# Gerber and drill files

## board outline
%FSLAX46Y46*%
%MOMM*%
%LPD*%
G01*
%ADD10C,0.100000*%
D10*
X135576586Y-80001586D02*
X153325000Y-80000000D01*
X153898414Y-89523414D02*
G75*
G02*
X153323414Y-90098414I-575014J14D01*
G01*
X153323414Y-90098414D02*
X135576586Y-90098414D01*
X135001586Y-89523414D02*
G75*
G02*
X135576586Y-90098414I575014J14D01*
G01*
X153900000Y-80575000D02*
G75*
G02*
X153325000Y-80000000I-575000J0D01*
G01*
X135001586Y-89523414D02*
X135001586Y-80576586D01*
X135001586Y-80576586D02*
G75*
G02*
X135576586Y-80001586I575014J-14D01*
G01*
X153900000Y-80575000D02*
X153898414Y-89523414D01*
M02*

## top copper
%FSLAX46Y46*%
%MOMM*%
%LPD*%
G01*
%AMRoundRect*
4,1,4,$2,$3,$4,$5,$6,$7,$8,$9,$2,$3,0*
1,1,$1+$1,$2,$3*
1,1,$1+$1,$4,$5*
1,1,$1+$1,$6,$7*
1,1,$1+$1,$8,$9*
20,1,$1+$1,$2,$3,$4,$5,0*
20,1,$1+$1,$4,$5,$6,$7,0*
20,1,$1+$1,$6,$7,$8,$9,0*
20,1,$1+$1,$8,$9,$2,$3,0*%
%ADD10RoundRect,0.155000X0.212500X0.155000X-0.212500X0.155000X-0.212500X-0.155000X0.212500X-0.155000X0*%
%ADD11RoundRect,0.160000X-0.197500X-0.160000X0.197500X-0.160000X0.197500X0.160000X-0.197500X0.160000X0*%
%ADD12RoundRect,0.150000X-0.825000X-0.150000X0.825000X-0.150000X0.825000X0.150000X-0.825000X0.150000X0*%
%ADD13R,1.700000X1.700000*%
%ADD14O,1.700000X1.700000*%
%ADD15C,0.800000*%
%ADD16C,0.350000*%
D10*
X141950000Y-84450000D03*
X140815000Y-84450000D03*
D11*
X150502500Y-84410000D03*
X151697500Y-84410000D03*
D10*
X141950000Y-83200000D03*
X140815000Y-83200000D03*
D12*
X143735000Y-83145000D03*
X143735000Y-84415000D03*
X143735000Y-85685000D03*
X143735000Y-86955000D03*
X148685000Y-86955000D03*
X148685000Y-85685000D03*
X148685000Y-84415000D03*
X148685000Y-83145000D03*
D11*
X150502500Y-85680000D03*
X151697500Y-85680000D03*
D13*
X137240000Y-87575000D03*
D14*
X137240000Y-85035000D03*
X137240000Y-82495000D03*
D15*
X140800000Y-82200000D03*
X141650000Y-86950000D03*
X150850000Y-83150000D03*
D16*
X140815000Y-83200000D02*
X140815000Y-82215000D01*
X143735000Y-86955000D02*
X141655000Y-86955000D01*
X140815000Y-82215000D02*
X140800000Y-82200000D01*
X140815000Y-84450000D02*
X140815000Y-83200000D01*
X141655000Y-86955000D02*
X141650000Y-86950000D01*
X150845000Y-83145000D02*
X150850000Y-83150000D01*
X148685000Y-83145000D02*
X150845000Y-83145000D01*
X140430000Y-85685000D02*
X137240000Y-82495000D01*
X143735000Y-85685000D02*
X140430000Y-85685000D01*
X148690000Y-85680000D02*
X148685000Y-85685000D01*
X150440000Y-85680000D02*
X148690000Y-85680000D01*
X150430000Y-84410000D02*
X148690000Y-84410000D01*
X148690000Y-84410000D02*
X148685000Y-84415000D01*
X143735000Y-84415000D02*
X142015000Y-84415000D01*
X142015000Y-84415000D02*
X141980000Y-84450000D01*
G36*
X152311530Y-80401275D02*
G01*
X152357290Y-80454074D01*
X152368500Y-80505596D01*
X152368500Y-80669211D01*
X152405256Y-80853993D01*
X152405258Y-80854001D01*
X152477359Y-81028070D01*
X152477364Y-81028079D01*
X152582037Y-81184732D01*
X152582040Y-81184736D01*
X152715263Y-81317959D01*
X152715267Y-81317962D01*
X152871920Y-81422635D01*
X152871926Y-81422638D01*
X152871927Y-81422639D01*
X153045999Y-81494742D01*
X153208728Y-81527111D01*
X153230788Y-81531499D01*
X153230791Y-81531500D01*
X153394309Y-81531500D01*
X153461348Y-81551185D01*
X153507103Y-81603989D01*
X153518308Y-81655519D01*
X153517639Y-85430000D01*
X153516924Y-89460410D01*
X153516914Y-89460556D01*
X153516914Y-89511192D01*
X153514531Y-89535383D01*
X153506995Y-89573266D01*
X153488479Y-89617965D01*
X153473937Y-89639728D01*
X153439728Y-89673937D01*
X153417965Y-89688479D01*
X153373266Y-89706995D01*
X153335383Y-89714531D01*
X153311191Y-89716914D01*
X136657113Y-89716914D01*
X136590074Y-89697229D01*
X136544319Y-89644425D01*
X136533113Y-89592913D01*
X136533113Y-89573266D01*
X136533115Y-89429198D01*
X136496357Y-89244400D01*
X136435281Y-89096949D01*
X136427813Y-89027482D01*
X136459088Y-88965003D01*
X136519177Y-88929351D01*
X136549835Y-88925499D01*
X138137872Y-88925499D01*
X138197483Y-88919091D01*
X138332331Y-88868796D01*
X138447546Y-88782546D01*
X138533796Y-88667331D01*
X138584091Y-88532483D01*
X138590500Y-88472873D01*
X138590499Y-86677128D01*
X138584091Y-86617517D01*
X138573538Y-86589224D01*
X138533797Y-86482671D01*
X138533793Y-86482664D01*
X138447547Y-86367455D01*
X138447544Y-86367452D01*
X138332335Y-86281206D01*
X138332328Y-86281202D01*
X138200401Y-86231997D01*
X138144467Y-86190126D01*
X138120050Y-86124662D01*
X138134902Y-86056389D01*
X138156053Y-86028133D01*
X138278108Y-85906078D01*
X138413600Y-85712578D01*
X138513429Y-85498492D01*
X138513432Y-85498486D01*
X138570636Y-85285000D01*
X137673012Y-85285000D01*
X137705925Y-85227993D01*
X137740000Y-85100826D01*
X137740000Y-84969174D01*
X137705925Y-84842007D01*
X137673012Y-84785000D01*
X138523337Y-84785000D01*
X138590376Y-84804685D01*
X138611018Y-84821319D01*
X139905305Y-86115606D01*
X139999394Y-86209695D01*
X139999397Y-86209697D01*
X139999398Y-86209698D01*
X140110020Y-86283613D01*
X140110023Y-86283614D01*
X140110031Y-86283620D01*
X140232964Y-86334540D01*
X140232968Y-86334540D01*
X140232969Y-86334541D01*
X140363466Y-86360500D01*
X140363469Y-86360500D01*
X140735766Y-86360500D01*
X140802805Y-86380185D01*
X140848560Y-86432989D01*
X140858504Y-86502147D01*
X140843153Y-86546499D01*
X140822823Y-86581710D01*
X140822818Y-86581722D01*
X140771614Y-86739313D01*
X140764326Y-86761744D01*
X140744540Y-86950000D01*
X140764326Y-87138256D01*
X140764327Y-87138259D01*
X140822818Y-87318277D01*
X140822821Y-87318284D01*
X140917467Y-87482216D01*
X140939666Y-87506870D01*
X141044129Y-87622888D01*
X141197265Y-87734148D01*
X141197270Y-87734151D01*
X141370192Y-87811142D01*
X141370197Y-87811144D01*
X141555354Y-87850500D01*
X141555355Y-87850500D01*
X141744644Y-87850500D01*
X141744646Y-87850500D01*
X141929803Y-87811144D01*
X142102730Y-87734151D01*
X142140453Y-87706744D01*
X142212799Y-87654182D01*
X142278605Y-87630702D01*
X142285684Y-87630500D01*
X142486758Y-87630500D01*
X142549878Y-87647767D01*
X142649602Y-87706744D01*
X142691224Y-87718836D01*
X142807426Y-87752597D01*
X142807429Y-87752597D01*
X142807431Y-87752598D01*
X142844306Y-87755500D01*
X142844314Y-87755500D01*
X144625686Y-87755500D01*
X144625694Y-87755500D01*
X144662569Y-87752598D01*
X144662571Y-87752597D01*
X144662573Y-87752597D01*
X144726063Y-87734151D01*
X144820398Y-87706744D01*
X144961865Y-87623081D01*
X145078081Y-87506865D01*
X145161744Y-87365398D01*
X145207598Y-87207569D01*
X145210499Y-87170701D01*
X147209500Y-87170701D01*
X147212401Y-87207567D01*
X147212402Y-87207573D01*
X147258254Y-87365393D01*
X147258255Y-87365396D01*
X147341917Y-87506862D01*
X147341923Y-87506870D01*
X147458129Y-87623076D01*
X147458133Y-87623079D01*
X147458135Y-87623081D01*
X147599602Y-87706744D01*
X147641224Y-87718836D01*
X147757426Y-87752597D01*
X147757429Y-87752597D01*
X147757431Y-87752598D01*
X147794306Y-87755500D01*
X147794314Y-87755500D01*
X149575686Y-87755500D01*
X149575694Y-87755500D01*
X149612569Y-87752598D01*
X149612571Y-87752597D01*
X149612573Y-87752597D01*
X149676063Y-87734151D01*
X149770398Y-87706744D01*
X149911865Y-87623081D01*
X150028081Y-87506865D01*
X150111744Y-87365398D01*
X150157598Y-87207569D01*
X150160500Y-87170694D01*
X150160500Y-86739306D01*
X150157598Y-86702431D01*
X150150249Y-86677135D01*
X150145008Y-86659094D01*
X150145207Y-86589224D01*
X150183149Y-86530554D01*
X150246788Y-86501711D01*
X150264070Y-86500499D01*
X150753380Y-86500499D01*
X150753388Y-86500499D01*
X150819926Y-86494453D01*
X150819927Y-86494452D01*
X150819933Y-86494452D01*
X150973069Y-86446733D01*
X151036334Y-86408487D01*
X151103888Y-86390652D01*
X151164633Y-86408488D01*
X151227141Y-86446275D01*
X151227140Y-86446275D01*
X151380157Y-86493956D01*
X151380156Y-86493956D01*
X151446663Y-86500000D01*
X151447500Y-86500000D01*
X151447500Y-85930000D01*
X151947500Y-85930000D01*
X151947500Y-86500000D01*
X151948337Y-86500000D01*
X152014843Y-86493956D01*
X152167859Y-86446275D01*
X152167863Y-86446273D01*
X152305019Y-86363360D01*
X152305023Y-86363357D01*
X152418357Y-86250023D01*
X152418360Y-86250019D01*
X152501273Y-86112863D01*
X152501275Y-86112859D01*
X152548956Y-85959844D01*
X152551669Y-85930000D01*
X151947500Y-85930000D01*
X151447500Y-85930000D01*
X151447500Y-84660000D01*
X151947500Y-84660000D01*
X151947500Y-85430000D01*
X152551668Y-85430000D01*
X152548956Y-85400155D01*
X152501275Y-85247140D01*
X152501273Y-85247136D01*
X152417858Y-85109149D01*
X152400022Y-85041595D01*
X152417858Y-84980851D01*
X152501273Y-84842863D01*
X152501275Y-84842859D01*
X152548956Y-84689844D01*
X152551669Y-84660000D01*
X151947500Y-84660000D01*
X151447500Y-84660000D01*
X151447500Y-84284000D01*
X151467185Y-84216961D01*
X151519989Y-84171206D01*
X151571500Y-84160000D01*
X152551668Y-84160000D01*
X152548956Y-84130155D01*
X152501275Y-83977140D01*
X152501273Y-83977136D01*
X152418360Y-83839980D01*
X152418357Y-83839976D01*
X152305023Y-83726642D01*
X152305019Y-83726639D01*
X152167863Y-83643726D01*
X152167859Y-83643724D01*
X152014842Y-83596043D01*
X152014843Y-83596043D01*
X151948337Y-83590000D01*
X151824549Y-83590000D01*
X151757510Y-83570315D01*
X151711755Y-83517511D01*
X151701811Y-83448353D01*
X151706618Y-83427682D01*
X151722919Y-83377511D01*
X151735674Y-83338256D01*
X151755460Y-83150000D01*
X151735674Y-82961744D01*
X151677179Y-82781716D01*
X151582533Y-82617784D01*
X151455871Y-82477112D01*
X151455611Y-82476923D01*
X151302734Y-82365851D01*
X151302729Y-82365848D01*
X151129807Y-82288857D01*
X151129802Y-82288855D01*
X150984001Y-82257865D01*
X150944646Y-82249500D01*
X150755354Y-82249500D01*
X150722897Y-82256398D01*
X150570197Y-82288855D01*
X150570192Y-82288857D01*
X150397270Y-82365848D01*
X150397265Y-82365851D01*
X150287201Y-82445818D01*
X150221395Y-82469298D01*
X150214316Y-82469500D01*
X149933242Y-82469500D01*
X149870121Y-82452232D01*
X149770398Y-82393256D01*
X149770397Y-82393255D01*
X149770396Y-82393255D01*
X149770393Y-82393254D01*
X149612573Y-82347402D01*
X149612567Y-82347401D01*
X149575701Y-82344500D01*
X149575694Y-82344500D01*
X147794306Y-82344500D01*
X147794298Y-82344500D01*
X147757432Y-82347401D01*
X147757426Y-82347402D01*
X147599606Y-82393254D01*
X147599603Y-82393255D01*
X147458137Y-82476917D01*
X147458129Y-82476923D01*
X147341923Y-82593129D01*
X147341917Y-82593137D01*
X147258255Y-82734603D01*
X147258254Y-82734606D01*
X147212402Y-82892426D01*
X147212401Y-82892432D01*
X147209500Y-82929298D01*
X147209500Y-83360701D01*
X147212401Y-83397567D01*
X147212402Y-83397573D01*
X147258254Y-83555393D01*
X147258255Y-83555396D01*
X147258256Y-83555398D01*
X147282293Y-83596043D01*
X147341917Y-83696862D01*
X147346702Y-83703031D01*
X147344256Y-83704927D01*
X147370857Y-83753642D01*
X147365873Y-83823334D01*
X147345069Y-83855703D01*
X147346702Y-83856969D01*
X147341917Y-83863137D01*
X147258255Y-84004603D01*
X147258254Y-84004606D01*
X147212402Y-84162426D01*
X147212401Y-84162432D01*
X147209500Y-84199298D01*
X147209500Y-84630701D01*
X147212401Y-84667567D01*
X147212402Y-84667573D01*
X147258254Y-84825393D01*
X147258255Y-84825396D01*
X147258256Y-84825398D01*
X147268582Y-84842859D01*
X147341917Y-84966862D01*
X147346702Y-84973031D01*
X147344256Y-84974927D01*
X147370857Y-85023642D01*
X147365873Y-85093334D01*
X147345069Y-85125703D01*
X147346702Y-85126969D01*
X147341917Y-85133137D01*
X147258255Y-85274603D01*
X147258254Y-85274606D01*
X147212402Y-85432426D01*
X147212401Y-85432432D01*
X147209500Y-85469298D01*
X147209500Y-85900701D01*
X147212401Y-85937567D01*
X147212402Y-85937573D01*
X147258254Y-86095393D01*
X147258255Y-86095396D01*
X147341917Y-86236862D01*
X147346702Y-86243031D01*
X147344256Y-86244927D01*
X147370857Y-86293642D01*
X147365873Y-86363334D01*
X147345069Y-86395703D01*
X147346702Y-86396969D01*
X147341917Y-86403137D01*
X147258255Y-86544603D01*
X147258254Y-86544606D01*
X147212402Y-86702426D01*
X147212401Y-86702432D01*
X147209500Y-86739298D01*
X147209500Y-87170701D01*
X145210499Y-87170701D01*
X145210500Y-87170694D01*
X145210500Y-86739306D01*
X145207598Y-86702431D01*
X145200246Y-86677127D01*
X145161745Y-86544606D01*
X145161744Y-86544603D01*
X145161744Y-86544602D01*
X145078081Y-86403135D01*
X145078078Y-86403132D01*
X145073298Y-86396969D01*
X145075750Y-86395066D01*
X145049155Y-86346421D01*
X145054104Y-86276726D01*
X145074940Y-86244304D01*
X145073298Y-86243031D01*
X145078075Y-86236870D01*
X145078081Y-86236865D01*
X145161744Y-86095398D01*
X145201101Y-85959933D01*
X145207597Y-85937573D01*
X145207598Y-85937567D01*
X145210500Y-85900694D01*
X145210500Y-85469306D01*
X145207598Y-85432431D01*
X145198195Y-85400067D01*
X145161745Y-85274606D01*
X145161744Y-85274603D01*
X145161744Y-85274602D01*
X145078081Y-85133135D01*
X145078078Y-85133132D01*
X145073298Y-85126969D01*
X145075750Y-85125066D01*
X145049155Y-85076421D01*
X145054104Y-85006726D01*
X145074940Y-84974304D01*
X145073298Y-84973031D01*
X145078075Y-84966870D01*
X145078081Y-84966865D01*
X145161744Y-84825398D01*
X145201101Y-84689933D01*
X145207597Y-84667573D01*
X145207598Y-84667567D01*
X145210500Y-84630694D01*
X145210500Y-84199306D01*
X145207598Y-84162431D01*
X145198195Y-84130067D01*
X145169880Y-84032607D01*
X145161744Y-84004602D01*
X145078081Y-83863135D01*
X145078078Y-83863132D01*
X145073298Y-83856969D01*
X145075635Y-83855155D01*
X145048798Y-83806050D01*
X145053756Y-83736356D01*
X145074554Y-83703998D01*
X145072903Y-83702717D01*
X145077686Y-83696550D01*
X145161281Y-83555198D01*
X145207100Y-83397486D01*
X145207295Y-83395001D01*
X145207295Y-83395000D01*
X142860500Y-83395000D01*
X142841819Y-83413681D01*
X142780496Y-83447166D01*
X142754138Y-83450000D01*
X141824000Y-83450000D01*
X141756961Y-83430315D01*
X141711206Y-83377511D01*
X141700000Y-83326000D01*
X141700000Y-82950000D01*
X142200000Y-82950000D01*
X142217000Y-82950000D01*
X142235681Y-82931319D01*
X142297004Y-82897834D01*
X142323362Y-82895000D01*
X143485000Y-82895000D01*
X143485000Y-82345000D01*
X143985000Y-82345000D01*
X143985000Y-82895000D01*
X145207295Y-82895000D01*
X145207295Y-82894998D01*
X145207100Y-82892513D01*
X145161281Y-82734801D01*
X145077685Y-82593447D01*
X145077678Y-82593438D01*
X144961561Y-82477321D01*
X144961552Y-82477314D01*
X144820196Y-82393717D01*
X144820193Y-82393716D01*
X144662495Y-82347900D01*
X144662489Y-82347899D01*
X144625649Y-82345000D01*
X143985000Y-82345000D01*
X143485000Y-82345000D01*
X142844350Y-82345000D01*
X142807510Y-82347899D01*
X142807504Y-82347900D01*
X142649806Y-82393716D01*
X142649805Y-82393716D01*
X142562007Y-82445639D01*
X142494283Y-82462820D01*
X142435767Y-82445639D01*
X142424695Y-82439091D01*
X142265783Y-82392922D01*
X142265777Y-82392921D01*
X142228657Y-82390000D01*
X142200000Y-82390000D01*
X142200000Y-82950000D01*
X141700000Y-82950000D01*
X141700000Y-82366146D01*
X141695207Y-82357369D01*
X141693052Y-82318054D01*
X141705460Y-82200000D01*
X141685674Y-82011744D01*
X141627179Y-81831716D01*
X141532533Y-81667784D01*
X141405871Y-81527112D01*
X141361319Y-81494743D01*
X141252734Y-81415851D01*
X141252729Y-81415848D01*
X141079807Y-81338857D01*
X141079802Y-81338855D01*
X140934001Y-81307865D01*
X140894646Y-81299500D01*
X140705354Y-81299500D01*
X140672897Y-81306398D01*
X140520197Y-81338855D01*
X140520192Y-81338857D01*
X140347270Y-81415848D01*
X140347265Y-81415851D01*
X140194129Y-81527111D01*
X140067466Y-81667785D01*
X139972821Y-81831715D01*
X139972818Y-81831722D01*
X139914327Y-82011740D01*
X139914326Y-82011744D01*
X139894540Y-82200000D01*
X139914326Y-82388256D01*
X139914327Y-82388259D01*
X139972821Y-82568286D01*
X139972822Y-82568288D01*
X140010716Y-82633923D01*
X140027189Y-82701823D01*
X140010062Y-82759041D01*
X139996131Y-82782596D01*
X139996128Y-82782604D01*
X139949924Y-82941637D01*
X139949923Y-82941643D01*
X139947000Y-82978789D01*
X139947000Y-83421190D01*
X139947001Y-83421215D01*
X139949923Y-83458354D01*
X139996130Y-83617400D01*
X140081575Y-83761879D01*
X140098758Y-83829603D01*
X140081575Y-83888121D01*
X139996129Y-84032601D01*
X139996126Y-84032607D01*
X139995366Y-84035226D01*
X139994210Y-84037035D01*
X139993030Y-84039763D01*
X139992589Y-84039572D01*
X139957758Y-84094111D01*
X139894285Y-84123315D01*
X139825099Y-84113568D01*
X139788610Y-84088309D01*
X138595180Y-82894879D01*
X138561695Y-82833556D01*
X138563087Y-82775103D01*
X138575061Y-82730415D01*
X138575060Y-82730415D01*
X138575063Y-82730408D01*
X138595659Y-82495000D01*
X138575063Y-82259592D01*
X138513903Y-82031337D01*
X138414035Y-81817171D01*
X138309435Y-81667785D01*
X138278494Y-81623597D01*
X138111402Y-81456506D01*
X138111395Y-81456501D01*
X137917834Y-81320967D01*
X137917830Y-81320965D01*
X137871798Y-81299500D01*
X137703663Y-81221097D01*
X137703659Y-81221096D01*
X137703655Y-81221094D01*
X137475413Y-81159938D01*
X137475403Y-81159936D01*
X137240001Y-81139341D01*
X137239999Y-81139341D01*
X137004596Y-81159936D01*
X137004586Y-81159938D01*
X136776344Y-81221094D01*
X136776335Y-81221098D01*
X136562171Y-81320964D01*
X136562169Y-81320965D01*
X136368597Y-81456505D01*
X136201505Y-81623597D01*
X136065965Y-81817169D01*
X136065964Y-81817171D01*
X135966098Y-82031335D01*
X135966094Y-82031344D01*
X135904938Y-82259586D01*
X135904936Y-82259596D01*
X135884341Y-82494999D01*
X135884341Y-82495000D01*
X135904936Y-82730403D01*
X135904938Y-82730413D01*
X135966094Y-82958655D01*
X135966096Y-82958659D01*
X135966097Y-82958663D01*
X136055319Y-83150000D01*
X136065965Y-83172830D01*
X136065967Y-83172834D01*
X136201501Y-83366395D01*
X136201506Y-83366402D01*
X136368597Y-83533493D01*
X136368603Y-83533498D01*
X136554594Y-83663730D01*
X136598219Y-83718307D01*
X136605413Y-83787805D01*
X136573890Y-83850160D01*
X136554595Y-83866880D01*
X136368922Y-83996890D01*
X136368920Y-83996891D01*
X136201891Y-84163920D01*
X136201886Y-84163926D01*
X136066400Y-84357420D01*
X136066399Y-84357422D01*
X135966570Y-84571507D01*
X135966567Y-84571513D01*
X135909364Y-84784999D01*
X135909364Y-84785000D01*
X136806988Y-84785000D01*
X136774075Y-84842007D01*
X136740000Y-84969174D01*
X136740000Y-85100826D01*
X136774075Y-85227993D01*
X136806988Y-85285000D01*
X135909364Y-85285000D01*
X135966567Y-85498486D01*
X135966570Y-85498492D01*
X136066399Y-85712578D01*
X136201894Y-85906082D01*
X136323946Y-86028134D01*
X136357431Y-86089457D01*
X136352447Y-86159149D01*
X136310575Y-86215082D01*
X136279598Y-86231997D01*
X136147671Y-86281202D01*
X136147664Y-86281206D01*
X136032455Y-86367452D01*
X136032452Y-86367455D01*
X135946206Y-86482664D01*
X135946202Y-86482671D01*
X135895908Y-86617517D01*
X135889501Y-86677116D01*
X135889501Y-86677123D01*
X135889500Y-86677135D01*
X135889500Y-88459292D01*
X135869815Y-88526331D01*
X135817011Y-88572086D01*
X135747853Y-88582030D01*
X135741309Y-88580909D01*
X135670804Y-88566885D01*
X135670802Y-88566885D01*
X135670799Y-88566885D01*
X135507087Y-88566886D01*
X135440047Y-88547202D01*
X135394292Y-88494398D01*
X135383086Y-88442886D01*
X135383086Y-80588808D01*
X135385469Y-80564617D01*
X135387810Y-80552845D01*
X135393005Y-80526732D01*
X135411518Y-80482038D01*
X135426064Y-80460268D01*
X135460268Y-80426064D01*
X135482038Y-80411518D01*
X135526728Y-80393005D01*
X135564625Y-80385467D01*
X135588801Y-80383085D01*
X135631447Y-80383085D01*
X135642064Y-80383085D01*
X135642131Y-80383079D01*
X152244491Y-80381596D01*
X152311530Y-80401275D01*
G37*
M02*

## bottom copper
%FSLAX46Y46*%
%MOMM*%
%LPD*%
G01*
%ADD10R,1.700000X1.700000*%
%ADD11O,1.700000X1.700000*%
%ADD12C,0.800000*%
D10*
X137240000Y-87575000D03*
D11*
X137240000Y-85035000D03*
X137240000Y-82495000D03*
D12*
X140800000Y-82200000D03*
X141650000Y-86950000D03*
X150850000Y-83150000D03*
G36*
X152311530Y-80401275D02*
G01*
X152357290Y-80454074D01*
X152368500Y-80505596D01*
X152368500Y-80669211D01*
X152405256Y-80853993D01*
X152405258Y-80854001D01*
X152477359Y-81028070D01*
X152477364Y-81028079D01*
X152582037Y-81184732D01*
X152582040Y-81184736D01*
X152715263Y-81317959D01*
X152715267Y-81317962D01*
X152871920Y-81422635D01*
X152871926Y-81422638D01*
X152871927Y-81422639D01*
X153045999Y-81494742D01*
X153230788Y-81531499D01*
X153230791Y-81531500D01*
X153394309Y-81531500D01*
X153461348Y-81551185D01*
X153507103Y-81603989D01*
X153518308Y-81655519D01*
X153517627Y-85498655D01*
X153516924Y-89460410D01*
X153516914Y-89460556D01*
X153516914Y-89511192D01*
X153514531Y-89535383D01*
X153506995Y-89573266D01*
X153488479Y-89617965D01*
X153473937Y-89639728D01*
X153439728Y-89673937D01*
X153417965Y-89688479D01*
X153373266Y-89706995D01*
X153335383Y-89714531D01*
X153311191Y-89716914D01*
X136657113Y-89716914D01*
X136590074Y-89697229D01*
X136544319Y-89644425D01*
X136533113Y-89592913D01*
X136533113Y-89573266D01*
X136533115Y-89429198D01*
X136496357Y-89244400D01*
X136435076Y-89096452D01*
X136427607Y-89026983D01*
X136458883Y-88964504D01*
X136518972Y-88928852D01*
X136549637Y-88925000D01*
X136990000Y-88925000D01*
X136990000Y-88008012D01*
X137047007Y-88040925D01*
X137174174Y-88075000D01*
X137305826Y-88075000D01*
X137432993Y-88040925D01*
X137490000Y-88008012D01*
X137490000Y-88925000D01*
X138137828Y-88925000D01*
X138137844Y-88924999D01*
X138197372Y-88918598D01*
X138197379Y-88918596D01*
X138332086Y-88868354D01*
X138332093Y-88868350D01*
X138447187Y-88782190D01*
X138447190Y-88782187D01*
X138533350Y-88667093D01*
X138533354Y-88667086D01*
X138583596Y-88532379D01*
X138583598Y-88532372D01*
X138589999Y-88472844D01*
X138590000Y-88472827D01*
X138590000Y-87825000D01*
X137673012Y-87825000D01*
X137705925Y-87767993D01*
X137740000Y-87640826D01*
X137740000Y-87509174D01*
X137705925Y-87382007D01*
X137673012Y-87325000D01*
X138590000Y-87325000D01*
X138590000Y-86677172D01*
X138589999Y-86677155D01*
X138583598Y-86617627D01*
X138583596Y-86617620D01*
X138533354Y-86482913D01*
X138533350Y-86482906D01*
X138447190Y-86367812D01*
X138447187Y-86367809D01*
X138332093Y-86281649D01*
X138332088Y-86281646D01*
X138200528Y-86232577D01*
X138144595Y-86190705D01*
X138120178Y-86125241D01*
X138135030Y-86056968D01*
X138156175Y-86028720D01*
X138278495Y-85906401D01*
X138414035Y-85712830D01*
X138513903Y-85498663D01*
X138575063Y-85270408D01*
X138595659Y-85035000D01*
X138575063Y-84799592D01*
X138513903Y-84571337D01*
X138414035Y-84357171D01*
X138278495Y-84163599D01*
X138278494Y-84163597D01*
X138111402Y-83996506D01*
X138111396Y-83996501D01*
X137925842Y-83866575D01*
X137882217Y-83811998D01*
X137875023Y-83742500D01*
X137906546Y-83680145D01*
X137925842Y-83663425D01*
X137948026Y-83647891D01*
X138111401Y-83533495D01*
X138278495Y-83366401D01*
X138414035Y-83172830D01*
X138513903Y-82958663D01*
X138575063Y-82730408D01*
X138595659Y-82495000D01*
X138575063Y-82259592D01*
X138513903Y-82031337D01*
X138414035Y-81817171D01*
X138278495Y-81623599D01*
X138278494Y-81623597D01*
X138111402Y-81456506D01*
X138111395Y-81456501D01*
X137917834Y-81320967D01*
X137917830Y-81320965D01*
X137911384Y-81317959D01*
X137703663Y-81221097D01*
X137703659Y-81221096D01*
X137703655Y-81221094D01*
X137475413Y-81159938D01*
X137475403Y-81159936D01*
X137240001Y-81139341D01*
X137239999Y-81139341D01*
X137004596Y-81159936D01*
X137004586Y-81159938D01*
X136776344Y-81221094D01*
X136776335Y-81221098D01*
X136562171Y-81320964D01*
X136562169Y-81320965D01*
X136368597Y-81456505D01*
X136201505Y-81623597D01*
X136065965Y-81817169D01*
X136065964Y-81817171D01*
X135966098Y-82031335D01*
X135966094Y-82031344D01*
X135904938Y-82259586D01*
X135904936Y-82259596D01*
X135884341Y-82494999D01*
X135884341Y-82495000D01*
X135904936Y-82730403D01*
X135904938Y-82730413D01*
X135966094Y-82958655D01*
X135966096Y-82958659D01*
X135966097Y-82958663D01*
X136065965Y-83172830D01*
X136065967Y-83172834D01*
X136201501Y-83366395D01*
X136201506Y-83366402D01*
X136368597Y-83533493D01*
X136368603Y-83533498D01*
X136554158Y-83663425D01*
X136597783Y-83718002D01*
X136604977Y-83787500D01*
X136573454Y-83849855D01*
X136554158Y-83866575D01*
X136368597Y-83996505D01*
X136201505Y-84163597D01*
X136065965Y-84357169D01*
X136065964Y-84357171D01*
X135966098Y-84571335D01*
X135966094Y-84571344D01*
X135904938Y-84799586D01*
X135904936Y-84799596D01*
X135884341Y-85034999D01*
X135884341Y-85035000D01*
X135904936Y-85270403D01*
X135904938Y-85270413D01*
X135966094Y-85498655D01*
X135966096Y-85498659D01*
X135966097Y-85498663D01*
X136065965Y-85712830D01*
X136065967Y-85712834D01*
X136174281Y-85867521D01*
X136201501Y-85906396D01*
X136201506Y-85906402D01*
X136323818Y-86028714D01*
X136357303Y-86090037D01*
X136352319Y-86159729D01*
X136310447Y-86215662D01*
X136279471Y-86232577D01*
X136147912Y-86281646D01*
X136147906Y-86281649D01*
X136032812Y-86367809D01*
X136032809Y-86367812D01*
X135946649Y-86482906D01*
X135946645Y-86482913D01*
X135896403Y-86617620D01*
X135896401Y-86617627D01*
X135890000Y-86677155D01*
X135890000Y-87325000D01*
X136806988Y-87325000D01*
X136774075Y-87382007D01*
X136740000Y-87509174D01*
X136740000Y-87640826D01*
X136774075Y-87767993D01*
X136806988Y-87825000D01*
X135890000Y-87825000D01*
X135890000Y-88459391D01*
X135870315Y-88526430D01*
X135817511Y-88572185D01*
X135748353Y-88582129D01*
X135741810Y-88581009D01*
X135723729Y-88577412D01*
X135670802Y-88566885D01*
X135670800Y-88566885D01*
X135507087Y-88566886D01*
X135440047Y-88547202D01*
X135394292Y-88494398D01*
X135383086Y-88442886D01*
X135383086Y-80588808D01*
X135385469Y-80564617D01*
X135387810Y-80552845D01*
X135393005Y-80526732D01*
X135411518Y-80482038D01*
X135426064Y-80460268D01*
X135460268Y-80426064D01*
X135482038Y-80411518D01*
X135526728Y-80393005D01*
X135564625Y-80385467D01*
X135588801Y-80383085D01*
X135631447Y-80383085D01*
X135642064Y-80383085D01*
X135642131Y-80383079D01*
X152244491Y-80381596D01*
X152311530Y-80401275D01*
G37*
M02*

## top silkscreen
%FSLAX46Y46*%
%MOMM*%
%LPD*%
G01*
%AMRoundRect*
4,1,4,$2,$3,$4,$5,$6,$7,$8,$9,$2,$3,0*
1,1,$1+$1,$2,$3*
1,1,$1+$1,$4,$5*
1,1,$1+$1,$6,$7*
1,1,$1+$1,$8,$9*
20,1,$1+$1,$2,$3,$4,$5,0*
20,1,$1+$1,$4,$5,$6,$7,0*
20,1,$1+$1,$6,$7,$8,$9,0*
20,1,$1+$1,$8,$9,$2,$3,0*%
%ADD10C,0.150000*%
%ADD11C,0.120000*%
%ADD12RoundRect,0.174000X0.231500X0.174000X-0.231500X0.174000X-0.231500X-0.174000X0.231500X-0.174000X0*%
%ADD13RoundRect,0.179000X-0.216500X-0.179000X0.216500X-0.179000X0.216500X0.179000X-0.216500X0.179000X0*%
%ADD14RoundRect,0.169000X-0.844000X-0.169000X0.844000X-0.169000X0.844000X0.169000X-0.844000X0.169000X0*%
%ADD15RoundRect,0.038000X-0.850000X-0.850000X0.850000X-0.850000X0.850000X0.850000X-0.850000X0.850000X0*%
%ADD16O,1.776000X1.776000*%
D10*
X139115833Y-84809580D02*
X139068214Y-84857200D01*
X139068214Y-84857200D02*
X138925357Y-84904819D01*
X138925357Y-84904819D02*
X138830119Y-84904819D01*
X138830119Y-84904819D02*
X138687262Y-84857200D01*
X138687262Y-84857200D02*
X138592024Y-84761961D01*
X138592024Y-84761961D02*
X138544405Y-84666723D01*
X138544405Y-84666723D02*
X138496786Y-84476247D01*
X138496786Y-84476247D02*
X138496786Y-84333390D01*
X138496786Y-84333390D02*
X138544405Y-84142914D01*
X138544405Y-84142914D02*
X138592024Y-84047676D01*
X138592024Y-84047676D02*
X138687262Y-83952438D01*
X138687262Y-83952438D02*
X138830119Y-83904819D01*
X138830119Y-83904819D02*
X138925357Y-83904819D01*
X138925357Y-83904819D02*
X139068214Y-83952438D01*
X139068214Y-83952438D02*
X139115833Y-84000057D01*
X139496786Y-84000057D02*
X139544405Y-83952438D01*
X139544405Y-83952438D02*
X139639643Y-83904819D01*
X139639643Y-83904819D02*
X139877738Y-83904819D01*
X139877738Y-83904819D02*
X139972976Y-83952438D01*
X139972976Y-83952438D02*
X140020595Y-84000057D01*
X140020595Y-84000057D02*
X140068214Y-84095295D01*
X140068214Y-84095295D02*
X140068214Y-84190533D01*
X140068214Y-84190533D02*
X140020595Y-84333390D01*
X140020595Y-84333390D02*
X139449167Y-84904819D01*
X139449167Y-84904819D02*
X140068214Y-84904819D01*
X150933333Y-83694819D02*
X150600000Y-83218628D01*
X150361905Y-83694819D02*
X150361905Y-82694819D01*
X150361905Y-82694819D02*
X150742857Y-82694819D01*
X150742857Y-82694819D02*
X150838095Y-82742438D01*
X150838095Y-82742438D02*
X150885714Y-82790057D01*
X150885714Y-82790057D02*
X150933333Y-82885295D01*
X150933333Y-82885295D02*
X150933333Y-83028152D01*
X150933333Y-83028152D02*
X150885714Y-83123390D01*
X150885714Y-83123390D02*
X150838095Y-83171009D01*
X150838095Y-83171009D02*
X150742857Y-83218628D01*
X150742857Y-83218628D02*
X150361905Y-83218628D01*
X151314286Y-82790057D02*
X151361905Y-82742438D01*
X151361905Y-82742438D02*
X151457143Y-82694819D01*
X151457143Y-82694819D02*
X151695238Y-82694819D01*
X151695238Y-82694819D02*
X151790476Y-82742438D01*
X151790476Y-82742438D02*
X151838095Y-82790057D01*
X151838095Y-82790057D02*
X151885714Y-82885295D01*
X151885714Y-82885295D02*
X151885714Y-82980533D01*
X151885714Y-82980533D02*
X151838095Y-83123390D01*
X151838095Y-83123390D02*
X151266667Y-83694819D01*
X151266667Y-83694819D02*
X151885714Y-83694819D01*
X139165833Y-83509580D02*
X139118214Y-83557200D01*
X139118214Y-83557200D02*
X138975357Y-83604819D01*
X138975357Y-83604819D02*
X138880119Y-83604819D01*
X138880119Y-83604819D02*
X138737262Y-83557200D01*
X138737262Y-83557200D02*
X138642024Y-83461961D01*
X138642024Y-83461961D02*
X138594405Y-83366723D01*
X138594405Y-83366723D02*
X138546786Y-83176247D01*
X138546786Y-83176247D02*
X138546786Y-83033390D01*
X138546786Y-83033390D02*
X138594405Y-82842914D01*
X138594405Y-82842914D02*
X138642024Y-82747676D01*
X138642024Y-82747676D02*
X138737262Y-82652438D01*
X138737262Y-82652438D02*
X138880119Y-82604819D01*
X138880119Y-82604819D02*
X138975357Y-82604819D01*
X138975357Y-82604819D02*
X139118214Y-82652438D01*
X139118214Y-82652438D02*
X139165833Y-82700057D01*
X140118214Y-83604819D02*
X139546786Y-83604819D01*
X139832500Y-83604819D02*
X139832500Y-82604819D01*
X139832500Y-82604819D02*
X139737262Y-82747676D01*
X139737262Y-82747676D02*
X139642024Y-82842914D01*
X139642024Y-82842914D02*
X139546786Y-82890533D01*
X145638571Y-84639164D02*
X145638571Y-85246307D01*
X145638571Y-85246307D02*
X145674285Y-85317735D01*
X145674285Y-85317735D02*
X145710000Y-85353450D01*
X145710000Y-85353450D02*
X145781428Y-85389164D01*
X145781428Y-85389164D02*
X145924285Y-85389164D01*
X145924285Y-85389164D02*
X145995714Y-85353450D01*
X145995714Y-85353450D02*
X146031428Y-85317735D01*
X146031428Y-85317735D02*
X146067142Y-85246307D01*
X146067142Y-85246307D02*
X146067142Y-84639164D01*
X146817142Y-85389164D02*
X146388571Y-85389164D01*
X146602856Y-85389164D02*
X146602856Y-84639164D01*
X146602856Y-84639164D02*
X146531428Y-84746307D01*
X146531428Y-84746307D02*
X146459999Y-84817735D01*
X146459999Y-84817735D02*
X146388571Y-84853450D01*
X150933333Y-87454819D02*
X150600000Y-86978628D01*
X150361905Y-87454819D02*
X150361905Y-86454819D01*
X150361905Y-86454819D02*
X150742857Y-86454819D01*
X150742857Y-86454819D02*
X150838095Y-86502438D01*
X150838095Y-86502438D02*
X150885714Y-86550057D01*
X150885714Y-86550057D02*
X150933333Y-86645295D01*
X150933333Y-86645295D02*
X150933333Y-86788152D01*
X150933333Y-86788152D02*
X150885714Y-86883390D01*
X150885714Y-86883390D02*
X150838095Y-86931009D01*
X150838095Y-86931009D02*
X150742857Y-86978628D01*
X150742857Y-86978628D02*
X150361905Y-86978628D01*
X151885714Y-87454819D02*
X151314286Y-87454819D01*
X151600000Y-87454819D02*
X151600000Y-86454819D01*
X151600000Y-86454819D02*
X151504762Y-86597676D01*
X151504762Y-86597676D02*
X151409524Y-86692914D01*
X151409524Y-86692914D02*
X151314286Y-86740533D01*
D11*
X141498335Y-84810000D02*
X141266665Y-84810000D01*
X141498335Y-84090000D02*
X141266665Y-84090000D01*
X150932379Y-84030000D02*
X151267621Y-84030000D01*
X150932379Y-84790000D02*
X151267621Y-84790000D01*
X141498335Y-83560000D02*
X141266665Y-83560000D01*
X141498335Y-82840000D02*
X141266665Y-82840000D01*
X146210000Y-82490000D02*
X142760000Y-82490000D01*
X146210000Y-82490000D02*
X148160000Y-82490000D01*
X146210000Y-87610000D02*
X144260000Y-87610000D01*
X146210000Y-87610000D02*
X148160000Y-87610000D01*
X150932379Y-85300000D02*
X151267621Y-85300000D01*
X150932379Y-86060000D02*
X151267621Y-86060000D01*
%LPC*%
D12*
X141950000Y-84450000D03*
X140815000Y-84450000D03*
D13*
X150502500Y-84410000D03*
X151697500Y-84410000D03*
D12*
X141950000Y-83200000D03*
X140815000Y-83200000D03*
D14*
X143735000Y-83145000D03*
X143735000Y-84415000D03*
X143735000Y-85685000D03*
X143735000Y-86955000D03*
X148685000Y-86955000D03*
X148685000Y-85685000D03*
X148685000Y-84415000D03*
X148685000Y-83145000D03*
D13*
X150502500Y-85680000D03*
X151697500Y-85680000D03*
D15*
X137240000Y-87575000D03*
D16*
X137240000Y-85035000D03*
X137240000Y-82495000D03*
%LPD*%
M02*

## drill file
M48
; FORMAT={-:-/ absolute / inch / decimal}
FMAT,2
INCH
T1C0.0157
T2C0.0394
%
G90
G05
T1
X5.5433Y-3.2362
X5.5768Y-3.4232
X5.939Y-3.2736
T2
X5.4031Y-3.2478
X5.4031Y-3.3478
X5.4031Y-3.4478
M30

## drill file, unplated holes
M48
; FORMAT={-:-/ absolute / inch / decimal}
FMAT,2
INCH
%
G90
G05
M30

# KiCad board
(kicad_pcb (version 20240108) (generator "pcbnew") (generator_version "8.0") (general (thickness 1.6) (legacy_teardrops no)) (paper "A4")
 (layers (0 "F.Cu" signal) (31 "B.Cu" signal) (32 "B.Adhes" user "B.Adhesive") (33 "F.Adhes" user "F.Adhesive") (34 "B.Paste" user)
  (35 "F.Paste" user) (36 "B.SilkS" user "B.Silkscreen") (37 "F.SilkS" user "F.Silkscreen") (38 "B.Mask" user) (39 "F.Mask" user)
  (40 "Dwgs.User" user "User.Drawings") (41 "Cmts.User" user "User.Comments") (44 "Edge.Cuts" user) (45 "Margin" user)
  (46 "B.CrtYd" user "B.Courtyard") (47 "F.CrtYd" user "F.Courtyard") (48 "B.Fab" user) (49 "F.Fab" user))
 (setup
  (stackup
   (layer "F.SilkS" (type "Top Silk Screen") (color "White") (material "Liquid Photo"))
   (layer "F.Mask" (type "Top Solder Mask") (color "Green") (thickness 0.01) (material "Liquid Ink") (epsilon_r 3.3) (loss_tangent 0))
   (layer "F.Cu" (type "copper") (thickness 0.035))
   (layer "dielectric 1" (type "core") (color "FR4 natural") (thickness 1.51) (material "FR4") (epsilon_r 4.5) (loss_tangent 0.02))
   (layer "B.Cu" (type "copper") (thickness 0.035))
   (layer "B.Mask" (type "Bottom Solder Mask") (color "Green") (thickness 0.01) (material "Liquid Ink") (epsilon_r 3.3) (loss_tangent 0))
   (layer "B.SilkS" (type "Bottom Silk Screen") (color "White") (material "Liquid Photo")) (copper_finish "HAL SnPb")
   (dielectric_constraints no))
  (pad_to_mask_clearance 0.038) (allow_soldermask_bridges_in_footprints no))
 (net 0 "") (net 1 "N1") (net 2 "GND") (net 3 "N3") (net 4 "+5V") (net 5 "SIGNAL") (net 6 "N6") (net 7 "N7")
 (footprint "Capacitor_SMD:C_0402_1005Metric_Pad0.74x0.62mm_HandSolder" (layer "F.Cu") (at 141.3825 84.45 180)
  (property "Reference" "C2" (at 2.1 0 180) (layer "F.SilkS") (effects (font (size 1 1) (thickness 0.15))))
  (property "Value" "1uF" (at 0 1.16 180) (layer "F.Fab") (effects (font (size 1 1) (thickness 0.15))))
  (fp_line (start -0.115835 0.36) (end 0.115835 0.36) (stroke (width 0.12) (type solid)) (layer "F.SilkS"))
  (fp_line (start -0.115835 -0.36) (end 0.115835 -0.36) (stroke (width 0.12) (type solid)) (layer "F.SilkS"))
  (pad "1" smd roundrect (at -0.5675 0 180) (size 0.735 0.62) (layers "F.Cu" "F.Paste" "F.Mask") (roundrect_rratio 0.25) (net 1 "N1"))
  (pad "2" smd roundrect (at 0.5675 0 180) (size 0.735 0.62) (layers "F.Cu" "F.Paste" "F.Mask") (roundrect_rratio 0.25) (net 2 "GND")))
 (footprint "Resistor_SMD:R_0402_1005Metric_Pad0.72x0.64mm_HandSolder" (layer "F.Cu") (at 151.1 84.41)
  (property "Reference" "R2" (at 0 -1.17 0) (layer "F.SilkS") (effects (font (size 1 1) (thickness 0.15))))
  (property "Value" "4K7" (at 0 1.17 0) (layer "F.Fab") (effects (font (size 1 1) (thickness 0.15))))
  (fp_line (start -0.167621 -0.38) (end 0.167621 -0.38) (stroke (width 0.12) (type solid)) (layer "F.SilkS"))
  (fp_line (start -0.167621 0.38) (end 0.167621 0.38) (stroke (width 0.12) (type solid)) (layer "F.SilkS"))
  (pad "1" smd roundrect (at -0.5975 0) (size 0.715 0.64) (layers "F.Cu" "F.Paste" "F.Mask") (roundrect_rratio 0.25) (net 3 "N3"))
  (pad "2" smd roundrect (at 0.5975 0) (size 0.715 0.64) (layers "F.Cu" "F.Paste" "F.Mask") (roundrect_rratio 0.25) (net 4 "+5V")))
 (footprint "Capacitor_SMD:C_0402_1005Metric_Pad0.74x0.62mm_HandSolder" (layer "F.Cu") (at 141.3825 83.2 180)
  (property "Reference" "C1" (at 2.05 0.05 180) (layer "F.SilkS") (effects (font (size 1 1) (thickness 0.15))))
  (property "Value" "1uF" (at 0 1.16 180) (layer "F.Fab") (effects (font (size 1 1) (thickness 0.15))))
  (fp_line (start -0.115835 0.36) (end 0.115835 0.36) (stroke (width 0.12) (type solid)) (layer "F.SilkS"))
  (fp_line (start -0.115835 -0.36) (end 0.115835 -0.36) (stroke (width 0.12) (type solid)) (layer "F.SilkS"))
  (pad "1" smd roundrect (at -0.5675 0 180) (size 0.735 0.62) (layers "F.Cu" "F.Paste" "F.Mask") (roundrect_rratio 0.25) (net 4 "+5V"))
  (pad "2" smd roundrect (at 0.5675 0 180) (size 0.735 0.62) (layers "F.Cu" "F.Paste" "F.Mask") (roundrect_rratio 0.25) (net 2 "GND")))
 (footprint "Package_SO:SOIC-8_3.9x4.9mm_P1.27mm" (layer "F.Cu") (at 146.21 85.05)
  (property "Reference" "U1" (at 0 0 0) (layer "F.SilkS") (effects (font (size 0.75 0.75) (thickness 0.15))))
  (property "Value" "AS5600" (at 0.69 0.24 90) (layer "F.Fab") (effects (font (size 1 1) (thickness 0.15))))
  (fp_line (start 0 -2.56) (end -3.45 -2.56) (stroke (width 0.12) (type solid)) (layer "F.SilkS"))
  (fp_line (start 0 -2.56) (end 1.95 -2.56) (stroke (width 0.12) (type solid)) (layer "F.SilkS"))
  (fp_line (start 0 2.56) (end -1.95 2.56) (stroke (width 0.12) (type solid)) (layer "F.SilkS"))
  (fp_line (start 0 2.56) (end 1.95 2.56) (stroke (width 0.12) (type solid)) (layer "F.SilkS"))
  (pad "1" smd roundrect (at -2.475 -1.905) (size 1.95 0.6) (layers "F.Cu" "F.Paste" "F.Mask") (roundrect_rratio 0.25) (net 4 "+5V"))
  (pad "2" smd roundrect (at -2.475 -0.635) (size 1.95 0.6) (layers "F.Cu" "F.Paste" "F.Mask") (roundrect_rratio 0.25) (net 1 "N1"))
  (pad "3" smd roundrect (at -2.475 0.635) (size 1.95 0.6) (layers "F.Cu" "F.Paste" "F.Mask") (roundrect_rratio 0.25) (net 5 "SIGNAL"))
  (pad "4" smd roundrect (at -2.475 1.905) (size 1.95 0.6) (layers "F.Cu" "F.Paste" "F.Mask") (roundrect_rratio 0.25) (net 2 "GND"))
  (pad "5" smd roundrect (at 2.475 1.905) (size 1.95 0.6) (layers "F.Cu" "F.Paste" "F.Mask") (roundrect_rratio 0.25) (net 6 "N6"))
  (pad "6" smd roundrect (at 2.475 0.635) (size 1.95 0.6) (layers "F.Cu" "F.Paste" "F.Mask") (roundrect_rratio 0.25) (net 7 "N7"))
  (pad "7" smd roundrect (at 2.475 -0.635) (size 1.95 0.6) (layers "F.Cu" "F.Paste" "F.Mask") (roundrect_rratio 0.25) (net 3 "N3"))
  (pad "8" smd roundrect (at 2.475 -1.905) (size 1.95 0.6) (layers "F.Cu" "F.Paste" "F.Mask") (roundrect_rratio 0.25) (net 2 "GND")))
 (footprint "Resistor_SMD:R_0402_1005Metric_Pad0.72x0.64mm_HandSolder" (layer "F.Cu") (at 151.1 85.68)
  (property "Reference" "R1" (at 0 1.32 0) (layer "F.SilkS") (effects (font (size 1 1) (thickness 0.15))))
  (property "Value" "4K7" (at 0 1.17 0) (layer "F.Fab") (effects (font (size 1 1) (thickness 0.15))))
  (fp_line (start -0.167621 -0.38) (end 0.167621 -0.38) (stroke (width 0.12) (type solid)) (layer "F.SilkS"))
  (fp_line (start -0.167621 0.38) (end 0.167621 0.38) (stroke (width 0.12) (type solid)) (layer "F.SilkS"))
  (pad "1" smd roundrect (at -0.5975 0) (size 0.715 0.64) (layers "F.Cu" "F.Paste" "F.Mask") (roundrect_rratio 0.25) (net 7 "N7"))
  (pad "2" smd roundrect (at 0.5975 0) (size 0.715 0.64) (layers "F.Cu" "F.Paste" "F.Mask") (roundrect_rratio 0.25) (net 4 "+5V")))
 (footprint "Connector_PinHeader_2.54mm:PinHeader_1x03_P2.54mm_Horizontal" (layer "B.Cu") (at 137.24 87.575)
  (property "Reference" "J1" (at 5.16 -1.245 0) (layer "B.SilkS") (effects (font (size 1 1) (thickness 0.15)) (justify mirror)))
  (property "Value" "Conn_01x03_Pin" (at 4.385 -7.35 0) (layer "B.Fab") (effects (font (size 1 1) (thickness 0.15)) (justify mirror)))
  (pad "1" thru_hole rect (at 0 0) (size 1.7 1.7) (drill 1) (layers "*.Cu" "*.Mask") (remove_unused_layers no) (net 2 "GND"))
  (pad "2" thru_hole oval (at 0 -2.54) (size 1.7 1.7) (drill 1) (layers "*.Cu" "*.Mask") (remove_unused_layers no) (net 4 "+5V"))
  (pad "3" thru_hole oval (at 0 -5.08) (size 1.7 1.7) (drill 1) (layers "*.Cu" "*.Mask") (remove_unused_layers no) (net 5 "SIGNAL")))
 (gr_line (start 135.576586 80.001586) (end 153.325 80) (stroke (width 0.1) (type default)) (layer "Edge.Cuts"))
 (gr_arc (start 153.898414 89.523414) (mid 153.73 89.93) (end 153.323414 90.098414) (stroke (width 0.1) (type default)) (layer "Edge.Cuts"))
 (gr_line (start 153.323414 90.098414) (end 135.576586 90.098414) (stroke (width 0.1) (type default)) (layer "Edge.Cuts"))
 (gr_arc (start 135.001586 89.523414) (mid 135.983174 89.116826) (end 135.576586 90.098414) (stroke (width 0.1) (type default))
  (layer "Edge.Cuts"))
 (gr_arc (start 153.9 80.575) (mid 152.918412 80.981588) (end 153.325 80) (stroke (width 0.1) (type default)) (layer "Edge.Cuts"))
 (gr_line (start 135.001586 89.523414) (end 135.001586 80.576586) (stroke (width 0.1) (type default)) (layer "Edge.Cuts"))
 (gr_arc (start 135.001586 80.576586) (mid 135.17 80.17) (end 135.576586 80.001586) (stroke (width 0.1) (type default)) (layer "Edge.Cuts"))
 (gr_line (start 153.9 80.575) (end 153.898414 89.523414) (stroke (width 0.1) (type default)) (layer "Edge.Cuts"))
 (segment (start 140.815 83.2) (end 140.815 82.215) (width 0.35) (layer "F.Cu") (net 2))
 (segment (start 143.735 86.955) (end 141.655 86.955) (width 0.35) (layer "F.Cu") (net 2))
 (segment (start 140.815 82.215) (end 140.8 82.2) (width 0.35) (layer "F.Cu") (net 2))
 (segment (start 140.815 84.45) (end 140.815 83.2) (width 0.35) (layer "F.Cu") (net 2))
 (segment (start 141.655 86.955) (end 141.65 86.95) (width 0.35) (layer "F.Cu") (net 2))
 (segment (start 150.845 83.145) (end 150.85 83.15) (width 0.35) (layer "F.Cu") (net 2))
 (segment (start 148.685 83.145) (end 150.845 83.145) (width 0.35) (layer "F.Cu") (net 2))
 (via (at 140.8 82.2) (size 0.8) (drill 0.4) (layers "F.Cu" "B.Cu") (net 2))
 (via (at 141.65 86.95) (size 0.8) (drill 0.4) (layers "F.Cu" "B.Cu") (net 2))
 (via (at 150.85 83.15) (size 0.8) (drill 0.4) (layers "F.Cu" "B.Cu") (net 2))
 (segment (start 140.43 85.685) (end 137.24 82.495) (width 0.35) (layer "F.Cu") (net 5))
 (segment (start 143.735 85.685) (end 140.43 85.685) (width 0.35) (layer "F.Cu") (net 5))
 (segment (start 148.69 85.68) (end 148.685 85.685) (width 0.35) (layer "F.Cu") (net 7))
 (segment (start 150.44 85.68) (end 148.69 85.68) (width 0.35) (layer "F.Cu") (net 7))
 (segment (start 150.43 84.41) (end 148.69 84.41) (width 0.35) (layer "F.Cu") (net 3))
 (segment (start 148.69 84.41) (end 148.685 84.415) (width 0.35) (layer "F.Cu") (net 3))
 (segment (start 143.735 84.415) (end 142.015 84.415) (width 0.35) (layer "F.Cu") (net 1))
 (segment (start 142.015 84.415) (end 141.98 84.45) (width 0.35) (layer "F.Cu") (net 1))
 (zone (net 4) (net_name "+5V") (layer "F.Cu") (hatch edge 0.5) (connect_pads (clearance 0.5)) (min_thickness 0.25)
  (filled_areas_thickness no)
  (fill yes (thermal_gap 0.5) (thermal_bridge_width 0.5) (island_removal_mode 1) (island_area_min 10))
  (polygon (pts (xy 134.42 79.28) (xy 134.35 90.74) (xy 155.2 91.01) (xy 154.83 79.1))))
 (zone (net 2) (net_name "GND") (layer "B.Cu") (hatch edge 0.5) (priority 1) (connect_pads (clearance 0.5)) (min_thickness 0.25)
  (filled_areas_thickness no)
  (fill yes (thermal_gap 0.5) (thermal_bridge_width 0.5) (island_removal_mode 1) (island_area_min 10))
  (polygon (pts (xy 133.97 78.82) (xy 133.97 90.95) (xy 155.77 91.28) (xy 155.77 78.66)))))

